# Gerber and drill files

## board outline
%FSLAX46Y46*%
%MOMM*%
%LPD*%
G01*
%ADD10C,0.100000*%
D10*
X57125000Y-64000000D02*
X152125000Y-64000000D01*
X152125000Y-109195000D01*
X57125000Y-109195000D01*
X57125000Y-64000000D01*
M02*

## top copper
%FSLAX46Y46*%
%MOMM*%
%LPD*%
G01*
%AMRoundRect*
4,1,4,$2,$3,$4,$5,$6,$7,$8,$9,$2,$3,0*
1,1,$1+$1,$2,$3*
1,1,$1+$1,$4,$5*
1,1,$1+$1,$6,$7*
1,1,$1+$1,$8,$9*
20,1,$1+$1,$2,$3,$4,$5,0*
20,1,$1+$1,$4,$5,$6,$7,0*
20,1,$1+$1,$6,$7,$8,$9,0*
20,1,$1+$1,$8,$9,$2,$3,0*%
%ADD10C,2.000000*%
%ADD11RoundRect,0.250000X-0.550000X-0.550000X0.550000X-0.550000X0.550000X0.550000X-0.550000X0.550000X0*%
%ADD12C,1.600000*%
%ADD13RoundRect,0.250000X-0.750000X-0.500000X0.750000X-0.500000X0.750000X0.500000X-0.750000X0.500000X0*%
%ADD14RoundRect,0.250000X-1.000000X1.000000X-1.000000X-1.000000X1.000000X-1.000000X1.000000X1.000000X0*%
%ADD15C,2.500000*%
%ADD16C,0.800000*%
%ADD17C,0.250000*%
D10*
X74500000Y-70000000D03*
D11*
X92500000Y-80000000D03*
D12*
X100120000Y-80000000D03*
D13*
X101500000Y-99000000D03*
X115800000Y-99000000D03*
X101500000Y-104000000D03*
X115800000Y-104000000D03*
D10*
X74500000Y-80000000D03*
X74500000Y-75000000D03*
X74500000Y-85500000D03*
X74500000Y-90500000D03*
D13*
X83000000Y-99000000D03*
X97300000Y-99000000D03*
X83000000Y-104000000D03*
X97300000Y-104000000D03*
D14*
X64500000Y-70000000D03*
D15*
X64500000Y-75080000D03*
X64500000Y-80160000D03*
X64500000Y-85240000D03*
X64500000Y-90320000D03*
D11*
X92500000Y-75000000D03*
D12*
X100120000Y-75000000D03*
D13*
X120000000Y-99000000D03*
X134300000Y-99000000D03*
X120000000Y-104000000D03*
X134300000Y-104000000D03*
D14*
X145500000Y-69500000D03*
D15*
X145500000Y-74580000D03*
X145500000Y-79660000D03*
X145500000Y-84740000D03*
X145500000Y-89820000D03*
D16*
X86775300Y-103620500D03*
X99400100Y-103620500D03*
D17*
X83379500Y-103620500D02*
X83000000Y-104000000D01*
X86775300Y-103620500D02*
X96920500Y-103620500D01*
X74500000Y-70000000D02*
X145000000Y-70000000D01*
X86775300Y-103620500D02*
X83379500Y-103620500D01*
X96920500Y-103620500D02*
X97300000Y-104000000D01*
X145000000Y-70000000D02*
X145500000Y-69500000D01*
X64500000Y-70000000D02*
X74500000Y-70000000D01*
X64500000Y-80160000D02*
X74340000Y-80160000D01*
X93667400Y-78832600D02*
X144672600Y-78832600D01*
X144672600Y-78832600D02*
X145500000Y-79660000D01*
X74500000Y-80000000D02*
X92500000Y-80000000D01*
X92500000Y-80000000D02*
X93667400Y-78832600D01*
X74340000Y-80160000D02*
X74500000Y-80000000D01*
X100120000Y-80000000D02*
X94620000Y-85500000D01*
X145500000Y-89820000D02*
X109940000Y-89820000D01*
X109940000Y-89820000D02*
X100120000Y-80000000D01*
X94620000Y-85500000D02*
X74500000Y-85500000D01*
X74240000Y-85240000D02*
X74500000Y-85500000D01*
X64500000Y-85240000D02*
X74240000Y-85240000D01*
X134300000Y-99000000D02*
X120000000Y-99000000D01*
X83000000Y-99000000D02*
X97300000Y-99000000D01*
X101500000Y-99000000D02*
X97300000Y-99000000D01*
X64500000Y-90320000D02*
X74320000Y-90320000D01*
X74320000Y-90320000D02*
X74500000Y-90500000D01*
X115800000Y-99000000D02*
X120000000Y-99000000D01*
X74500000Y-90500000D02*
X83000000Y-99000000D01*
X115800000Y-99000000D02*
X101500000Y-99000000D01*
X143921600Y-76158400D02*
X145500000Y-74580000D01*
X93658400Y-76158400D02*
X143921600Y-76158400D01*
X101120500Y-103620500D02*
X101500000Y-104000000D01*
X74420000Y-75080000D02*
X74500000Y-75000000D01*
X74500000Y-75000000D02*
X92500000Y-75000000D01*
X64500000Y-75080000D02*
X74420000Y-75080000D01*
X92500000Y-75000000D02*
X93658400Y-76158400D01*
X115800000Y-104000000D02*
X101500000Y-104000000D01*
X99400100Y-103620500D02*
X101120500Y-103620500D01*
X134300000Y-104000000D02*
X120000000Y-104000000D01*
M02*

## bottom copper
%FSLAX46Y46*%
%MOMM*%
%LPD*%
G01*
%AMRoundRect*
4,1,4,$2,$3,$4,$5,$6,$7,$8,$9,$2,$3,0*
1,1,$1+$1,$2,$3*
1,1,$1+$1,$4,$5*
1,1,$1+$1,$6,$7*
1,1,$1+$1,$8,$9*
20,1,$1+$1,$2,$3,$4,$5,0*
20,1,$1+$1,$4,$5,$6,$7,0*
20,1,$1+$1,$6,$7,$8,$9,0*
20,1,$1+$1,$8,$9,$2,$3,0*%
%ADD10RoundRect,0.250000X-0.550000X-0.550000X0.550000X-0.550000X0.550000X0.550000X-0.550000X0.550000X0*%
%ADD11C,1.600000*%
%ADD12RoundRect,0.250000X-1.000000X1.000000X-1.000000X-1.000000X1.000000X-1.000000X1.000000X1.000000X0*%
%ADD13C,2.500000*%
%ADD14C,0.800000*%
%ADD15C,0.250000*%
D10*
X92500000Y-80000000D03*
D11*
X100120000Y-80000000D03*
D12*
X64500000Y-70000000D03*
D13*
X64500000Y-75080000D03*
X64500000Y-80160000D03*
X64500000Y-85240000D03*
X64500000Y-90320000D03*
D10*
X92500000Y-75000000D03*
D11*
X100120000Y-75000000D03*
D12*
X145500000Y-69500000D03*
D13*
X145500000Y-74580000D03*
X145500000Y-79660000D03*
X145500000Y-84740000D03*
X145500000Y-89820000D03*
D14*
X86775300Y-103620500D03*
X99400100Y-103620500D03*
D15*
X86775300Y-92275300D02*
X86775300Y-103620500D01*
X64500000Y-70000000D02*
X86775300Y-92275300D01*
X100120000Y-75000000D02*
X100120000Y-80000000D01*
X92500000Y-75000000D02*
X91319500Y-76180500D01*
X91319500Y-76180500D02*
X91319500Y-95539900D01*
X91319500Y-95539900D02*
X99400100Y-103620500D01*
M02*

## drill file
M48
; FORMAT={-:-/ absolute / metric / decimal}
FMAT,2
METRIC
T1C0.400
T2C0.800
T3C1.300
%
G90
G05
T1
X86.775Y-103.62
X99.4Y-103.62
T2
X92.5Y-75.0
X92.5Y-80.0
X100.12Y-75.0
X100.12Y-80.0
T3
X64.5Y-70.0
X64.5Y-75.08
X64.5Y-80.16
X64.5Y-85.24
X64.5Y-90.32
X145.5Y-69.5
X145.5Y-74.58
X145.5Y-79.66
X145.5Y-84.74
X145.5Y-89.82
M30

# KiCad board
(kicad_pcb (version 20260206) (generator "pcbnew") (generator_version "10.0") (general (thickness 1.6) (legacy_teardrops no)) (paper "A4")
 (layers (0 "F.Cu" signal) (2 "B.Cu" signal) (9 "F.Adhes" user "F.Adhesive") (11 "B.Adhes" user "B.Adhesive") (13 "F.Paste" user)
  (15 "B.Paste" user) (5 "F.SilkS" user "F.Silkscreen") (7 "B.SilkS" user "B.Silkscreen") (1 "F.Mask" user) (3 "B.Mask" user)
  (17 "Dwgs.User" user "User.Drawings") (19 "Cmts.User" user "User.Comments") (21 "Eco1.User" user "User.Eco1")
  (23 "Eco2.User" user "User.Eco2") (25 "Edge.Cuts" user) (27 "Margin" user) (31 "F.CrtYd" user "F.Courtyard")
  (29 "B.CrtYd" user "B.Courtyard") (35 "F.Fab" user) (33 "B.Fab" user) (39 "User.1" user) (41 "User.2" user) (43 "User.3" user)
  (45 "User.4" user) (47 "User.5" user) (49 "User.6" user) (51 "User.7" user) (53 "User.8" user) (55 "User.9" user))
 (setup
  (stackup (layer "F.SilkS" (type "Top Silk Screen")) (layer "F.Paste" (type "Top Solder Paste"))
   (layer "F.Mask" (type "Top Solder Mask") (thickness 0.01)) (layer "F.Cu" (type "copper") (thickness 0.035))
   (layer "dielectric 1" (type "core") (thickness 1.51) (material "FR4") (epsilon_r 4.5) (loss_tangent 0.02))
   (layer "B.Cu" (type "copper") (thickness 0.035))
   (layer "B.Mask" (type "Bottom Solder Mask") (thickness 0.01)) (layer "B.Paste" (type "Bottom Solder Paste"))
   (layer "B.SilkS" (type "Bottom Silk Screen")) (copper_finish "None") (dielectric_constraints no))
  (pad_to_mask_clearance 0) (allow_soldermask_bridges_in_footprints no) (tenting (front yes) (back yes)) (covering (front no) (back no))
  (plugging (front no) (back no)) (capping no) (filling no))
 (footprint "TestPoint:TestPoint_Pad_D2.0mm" (layer "F.Cu") (at 74.5 70)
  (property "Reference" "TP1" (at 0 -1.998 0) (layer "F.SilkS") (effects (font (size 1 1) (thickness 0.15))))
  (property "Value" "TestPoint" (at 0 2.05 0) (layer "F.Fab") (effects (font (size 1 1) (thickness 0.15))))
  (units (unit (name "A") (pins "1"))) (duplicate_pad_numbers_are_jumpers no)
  (pad "1" smd circle (at 0 0) (size 2 2) (layers "F.Cu" "F.Mask") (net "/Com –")))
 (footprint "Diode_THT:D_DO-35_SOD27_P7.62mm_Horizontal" (layer "F.Cu") (at 92.5 80)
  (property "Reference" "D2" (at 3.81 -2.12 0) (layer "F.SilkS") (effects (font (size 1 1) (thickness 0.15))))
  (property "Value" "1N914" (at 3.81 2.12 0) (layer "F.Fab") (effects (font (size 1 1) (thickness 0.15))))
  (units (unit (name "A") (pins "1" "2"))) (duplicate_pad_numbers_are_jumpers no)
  (pad "1" thru_hole roundrect (at 0 0) (size 1.6 1.6) (drill 0.8) (layers "*.Cu" "*.Mask") (remove_unused_layers no)
   (roundrect_rratio 0.15625) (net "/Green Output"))
  (pad "2" thru_hole circle (at 7.62 0) (size 1.6 1.6) (drill 0.8) (layers "*.Cu" "*.Mask") (remove_unused_layers no) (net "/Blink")))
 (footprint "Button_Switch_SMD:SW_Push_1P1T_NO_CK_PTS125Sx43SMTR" (layer "F.Cu") (at 108.65 101.5)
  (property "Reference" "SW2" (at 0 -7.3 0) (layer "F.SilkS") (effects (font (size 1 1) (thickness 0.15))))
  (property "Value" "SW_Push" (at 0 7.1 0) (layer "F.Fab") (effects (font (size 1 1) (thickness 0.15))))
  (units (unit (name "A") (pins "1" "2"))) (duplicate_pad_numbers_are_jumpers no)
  (pad "1" smd roundrect (at -7.15 -2.5) (size 2 1.5) (layers "F.Cu" "F.Mask" "F.Paste") (roundrect_rratio 0.1666666667)
   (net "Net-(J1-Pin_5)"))
  (pad "1" smd roundrect (at 7.15 -2.5) (size 2 1.5) (layers "F.Cu" "F.Mask" "F.Paste") (roundrect_rratio 0.1666666667)
   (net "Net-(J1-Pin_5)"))
  (pad "2" smd roundrect (at -7.15 2.5) (size 2 1.5) (layers "F.Cu" "F.Mask" "F.Paste") (roundrect_rratio 0.1666666667) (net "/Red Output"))
  (pad "2" smd roundrect (at 7.15 2.5) (size 2 1.5) (layers "F.Cu" "F.Mask" "F.Paste") (roundrect_rratio 0.1666666667) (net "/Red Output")))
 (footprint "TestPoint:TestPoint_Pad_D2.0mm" (layer "F.Cu") (at 74.5 80)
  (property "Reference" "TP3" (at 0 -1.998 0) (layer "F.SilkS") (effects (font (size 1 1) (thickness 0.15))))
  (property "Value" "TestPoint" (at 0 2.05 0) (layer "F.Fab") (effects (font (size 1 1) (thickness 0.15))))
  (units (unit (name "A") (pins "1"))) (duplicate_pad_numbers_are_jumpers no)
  (pad "1" smd circle (at 0 0) (size 2 2) (layers "F.Cu" "F.Mask") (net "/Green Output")))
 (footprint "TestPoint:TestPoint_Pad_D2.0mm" (layer "F.Cu") (at 74.5 75)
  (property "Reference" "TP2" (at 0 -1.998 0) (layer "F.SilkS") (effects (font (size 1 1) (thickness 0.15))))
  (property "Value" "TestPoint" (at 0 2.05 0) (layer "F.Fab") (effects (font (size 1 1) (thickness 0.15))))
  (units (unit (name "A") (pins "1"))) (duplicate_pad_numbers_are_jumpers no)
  (pad "1" smd circle (at 0 0) (size 2 2) (layers "F.Cu" "F.Mask") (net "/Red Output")))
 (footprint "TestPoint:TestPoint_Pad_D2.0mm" (layer "F.Cu") (at 74.5 85.5)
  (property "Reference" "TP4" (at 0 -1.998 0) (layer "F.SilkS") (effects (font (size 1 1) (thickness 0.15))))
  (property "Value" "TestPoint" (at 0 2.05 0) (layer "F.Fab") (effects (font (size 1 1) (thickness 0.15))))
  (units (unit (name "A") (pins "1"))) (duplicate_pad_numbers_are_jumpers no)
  (pad "1" smd circle (at 0 0) (size 2 2) (layers "F.Cu" "F.Mask") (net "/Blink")))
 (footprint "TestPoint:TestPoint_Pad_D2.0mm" (layer "F.Cu") (at 74.5 90.5)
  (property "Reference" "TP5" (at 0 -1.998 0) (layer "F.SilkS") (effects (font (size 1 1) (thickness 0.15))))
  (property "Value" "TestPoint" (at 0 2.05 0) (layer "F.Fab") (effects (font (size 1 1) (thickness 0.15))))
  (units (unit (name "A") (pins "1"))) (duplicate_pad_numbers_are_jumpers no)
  (pad "1" smd circle (at 0 0) (size 2 2) (layers "F.Cu" "F.Mask") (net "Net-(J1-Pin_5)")))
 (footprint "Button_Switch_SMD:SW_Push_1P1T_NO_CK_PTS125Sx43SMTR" (layer "F.Cu") (at 90.15 101.5)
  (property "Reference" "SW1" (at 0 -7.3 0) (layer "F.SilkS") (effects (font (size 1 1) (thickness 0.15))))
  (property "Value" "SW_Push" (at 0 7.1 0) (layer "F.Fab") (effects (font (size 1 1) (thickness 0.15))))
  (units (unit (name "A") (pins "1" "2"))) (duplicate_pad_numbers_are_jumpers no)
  (pad "1" smd roundrect (at -7.15 -2.5) (size 2 1.5) (layers "F.Cu" "F.Mask" "F.Paste") (roundrect_rratio 0.1666666667)
   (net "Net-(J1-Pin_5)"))
  (pad "1" smd roundrect (at 7.15 -2.5) (size 2 1.5) (layers "F.Cu" "F.Mask" "F.Paste") (roundrect_rratio 0.1666666667)
   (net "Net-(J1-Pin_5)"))
  (pad "2" smd roundrect (at -7.15 2.5) (size 2 1.5) (layers "F.Cu" "F.Mask" "F.Paste") (roundrect_rratio 0.1666666667) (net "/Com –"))
  (pad "2" smd roundrect (at 7.15 2.5) (size 2 1.5) (layers "F.Cu" "F.Mask" "F.Paste") (roundrect_rratio 0.1666666667) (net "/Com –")))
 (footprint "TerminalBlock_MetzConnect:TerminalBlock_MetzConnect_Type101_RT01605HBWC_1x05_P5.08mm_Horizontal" (layer "F.Cu")
  (at 64.5 70 -90)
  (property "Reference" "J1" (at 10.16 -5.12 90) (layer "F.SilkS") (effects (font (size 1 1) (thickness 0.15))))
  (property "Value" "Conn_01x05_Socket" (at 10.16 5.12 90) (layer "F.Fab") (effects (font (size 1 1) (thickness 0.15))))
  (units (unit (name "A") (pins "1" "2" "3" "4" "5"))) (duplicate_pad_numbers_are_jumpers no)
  (pad "1" thru_hole roundrect (at 0 0 270) (size 2.5 2.5) (drill 1.3) (layers "*.Cu" "*.Mask") (remove_unused_layers no)
   (roundrect_rratio 0.1) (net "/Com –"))
  (pad "2" thru_hole circle (at 5.08 0 270) (size 2.5 2.5) (drill 1.3) (layers "*.Cu" "*.Mask") (remove_unused_layers no)
   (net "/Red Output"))
  (pad "3" thru_hole circle (at 10.16 0 270) (size 2.5 2.5) (drill 1.3) (layers "*.Cu" "*.Mask") (remove_unused_layers no)
   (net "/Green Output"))
  (pad "4" thru_hole circle (at 15.24 0 270) (size 2.5 2.5) (drill 1.3) (layers "*.Cu" "*.Mask") (remove_unused_layers no) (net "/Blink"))
  (pad "5" thru_hole circle (at 20.32 0 270) (size 2.5 2.5) (drill 1.3) (layers "*.Cu" "*.Mask") (remove_unused_layers no)
   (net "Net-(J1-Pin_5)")))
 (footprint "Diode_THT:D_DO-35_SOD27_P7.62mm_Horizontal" (layer "F.Cu") (at 92.5 75)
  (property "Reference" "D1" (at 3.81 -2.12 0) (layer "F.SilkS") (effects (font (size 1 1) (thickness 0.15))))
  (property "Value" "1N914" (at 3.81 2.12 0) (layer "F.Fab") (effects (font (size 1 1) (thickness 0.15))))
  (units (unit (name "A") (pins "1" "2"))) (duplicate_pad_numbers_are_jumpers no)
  (pad "1" thru_hole roundrect (at 0 0) (size 1.6 1.6) (drill 0.8) (layers "*.Cu" "*.Mask") (remove_unused_layers no)
   (roundrect_rratio 0.15625) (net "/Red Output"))
  (pad "2" thru_hole circle (at 7.62 0) (size 1.6 1.6) (drill 0.8) (layers "*.Cu" "*.Mask") (remove_unused_layers no) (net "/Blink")))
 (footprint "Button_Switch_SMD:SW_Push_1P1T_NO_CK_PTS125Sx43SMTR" (layer "F.Cu") (at 127.15 101.5)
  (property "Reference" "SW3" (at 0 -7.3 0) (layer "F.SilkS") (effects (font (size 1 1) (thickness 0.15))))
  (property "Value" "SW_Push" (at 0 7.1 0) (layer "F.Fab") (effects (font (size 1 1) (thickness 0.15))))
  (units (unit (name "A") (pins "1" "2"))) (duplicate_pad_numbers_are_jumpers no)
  (pad "1" smd roundrect (at -7.15 -2.5) (size 2 1.5) (layers "F.Cu" "F.Mask" "F.Paste") (roundrect_rratio 0.1666666667)
   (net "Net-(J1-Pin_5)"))
  (pad "1" smd roundrect (at 7.15 -2.5) (size 2 1.5) (layers "F.Cu" "F.Mask" "F.Paste") (roundrect_rratio 0.1666666667)
   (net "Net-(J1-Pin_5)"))
  (pad "2" smd roundrect (at -7.15 2.5) (size 2 1.5) (layers "F.Cu" "F.Mask" "F.Paste") (roundrect_rratio 0.1666666667)
   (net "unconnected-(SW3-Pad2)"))
  (pad "2" smd roundrect (at 7.15 2.5) (size 2 1.5) (layers "F.Cu" "F.Mask" "F.Paste") (roundrect_rratio 0.1666666667)
   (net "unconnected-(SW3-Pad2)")))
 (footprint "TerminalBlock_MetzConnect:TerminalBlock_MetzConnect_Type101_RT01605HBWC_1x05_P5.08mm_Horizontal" (layer "F.Cu")
  (at 145.5 69.5 -90)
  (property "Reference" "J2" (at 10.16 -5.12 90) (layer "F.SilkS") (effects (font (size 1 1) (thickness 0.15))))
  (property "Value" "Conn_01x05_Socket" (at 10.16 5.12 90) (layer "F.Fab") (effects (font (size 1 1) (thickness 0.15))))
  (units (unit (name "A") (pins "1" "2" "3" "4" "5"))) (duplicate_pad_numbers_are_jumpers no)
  (pad "1" thru_hole roundrect (at 0 0 270) (size 2.5 2.5) (drill 1.3) (layers "*.Cu" "*.Mask") (remove_unused_layers no)
   (roundrect_rratio 0.1) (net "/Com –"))
  (pad "2" thru_hole circle (at 5.08 0 270) (size 2.5 2.5) (drill 1.3) (layers "*.Cu" "*.Mask") (remove_unused_layers no)
   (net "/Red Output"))
  (pad "3" thru_hole circle (at 10.16 0 270) (size 2.5 2.5) (drill 1.3) (layers "*.Cu" "*.Mask") (remove_unused_layers no)
   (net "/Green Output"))
  (pad "4" thru_hole circle (at 15.24 0 270) (size 2.5 2.5) (drill 1.3) (layers "*.Cu" "*.Mask") (remove_unused_layers no)
   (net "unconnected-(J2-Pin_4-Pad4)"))
  (pad "5" thru_hole circle (at 20.32 0 270) (size 2.5 2.5) (drill 1.3) (layers "*.Cu" "*.Mask") (remove_unused_layers no) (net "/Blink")))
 (gr_rect (start 57.125 64) (end 152.125 109.195) (stroke (width 0.1) (type default)) (fill no) (layer "Edge.Cuts"))
 (segment (start 83.3795 103.6205) (end 83 104) (width 0.25) (layer "F.Cu") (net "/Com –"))
 (segment (start 86.7753 103.6205) (end 96.9205 103.6205) (width 0.25) (layer "F.Cu") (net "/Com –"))
 (segment (start 74.5 70) (end 145 70) (width 0.25) (layer "F.Cu") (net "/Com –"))
 (segment (start 86.7753 103.6205) (end 83.3795 103.6205) (width 0.25) (layer "F.Cu") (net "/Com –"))
 (segment (start 96.9205 103.6205) (end 97.3 104) (width 0.25) (layer "F.Cu") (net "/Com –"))
 (segment (start 145 70) (end 145.5 69.5) (width 0.25) (layer "F.Cu") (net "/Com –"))
 (segment (start 64.5 70) (end 74.5 70) (width 0.25) (layer "F.Cu") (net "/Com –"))
 (via (at 86.7753 103.6205) (size 0.8) (drill 0.4) (layers "F.Cu" "B.Cu") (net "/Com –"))
 (segment (start 86.7753 92.2753) (end 86.7753 103.6205) (width 0.25) (layer "B.Cu") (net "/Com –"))
 (segment (start 64.5 70) (end 86.7753 92.2753) (width 0.25) (layer "B.Cu") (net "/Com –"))
 (segment (start 64.5 80.16) (end 74.34 80.16) (width 0.25) (layer "F.Cu") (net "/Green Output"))
 (segment (start 93.6674 78.8326) (end 144.6726 78.8326) (width 0.25) (layer "F.Cu") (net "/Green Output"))
 (segment (start 144.6726 78.8326) (end 145.5 79.66) (width 0.25) (layer "F.Cu") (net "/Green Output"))
 (segment (start 74.5 80) (end 92.5 80) (width 0.25) (layer "F.Cu") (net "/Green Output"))
 (segment (start 92.5 80) (end 93.6674 78.8326) (width 0.25) (layer "F.Cu") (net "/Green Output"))
 (segment (start 74.34 80.16) (end 74.5 80) (width 0.25) (layer "F.Cu") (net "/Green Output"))
 (segment (start 100.12 80) (end 94.62 85.5) (width 0.25) (layer "F.Cu") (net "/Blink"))
 (segment (start 145.5 89.82) (end 109.94 89.82) (width 0.25) (layer "F.Cu") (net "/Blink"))
 (segment (start 109.94 89.82) (end 100.12 80) (width 0.25) (layer "F.Cu") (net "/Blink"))
 (segment (start 94.62 85.5) (end 74.5 85.5) (width 0.25) (layer "F.Cu") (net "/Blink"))
 (segment (start 74.24 85.24) (end 74.5 85.5) (width 0.25) (layer "F.Cu") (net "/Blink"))
 (segment (start 64.5 85.24) (end 74.24 85.24) (width 0.25) (layer "F.Cu") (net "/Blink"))
 (segment (start 100.12 75) (end 100.12 80) (width 0.25) (layer "B.Cu") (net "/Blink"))
 (segment (start 134.3 99) (end 120 99) (width 0.25) (layer "F.Cu") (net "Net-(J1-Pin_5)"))
 (segment (start 83 99) (end 97.3 99) (width 0.25) (layer "F.Cu") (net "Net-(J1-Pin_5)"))
 (segment (start 101.5 99) (end 97.3 99) (width 0.25) (layer "F.Cu") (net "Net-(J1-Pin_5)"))
 (segment (start 64.5 90.32) (end 74.32 90.32) (width 0.25) (layer "F.Cu") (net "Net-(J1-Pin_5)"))
 (segment (start 74.32 90.32) (end 74.5 90.5) (width 0.25) (layer "F.Cu") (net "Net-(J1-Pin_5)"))
 (segment (start 115.8 99) (end 120 99) (width 0.25) (layer "F.Cu") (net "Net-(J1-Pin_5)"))
 (segment (start 74.5 90.5) (end 83 99) (width 0.25) (layer "F.Cu") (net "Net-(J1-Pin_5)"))
 (segment (start 115.8 99) (end 101.5 99) (width 0.25) (layer "F.Cu") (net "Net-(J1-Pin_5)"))
 (segment (start 143.9216 76.1584) (end 145.5 74.58) (width 0.25) (layer "F.Cu") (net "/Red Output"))
 (segment (start 93.6584 76.1584) (end 143.9216 76.1584) (width 0.25) (layer "F.Cu") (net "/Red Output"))
 (segment (start 101.1205 103.6205) (end 101.5 104) (width 0.25) (layer "F.Cu") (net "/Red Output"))
 (segment (start 74.42 75.08) (end 74.5 75) (width 0.25) (layer "F.Cu") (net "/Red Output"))
 (segment (start 74.5 75) (end 92.5 75) (width 0.25) (layer "F.Cu") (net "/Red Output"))
 (segment (start 64.5 75.08) (end 74.42 75.08) (width 0.25) (layer "F.Cu") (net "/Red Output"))
 (segment (start 92.5 75) (end 93.6584 76.1584) (width 0.25) (layer "F.Cu") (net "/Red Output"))
 (segment (start 115.8 104) (end 101.5 104) (width 0.25) (layer "F.Cu") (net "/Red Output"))
 (segment (start 99.4001 103.6205) (end 101.1205 103.6205) (width 0.25) (layer "F.Cu") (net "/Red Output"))
 (via (at 99.4001 103.6205) (size 0.8) (drill 0.4) (layers "F.Cu" "B.Cu") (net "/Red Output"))
 (segment (start 92.5 75) (end 91.3195 76.1805) (width 0.25) (layer "B.Cu") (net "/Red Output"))
 (segment (start 91.3195 76.1805) (end 91.3195 95.5399) (width 0.25) (layer "B.Cu") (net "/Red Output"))
 (segment (start 91.3195 95.5399) (end 99.4001 103.6205) (width 0.25) (layer "B.Cu") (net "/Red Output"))
 (segment (start 134.3 104) (end 120 104) (width 0.25) (layer "F.Cu") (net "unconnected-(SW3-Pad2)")))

